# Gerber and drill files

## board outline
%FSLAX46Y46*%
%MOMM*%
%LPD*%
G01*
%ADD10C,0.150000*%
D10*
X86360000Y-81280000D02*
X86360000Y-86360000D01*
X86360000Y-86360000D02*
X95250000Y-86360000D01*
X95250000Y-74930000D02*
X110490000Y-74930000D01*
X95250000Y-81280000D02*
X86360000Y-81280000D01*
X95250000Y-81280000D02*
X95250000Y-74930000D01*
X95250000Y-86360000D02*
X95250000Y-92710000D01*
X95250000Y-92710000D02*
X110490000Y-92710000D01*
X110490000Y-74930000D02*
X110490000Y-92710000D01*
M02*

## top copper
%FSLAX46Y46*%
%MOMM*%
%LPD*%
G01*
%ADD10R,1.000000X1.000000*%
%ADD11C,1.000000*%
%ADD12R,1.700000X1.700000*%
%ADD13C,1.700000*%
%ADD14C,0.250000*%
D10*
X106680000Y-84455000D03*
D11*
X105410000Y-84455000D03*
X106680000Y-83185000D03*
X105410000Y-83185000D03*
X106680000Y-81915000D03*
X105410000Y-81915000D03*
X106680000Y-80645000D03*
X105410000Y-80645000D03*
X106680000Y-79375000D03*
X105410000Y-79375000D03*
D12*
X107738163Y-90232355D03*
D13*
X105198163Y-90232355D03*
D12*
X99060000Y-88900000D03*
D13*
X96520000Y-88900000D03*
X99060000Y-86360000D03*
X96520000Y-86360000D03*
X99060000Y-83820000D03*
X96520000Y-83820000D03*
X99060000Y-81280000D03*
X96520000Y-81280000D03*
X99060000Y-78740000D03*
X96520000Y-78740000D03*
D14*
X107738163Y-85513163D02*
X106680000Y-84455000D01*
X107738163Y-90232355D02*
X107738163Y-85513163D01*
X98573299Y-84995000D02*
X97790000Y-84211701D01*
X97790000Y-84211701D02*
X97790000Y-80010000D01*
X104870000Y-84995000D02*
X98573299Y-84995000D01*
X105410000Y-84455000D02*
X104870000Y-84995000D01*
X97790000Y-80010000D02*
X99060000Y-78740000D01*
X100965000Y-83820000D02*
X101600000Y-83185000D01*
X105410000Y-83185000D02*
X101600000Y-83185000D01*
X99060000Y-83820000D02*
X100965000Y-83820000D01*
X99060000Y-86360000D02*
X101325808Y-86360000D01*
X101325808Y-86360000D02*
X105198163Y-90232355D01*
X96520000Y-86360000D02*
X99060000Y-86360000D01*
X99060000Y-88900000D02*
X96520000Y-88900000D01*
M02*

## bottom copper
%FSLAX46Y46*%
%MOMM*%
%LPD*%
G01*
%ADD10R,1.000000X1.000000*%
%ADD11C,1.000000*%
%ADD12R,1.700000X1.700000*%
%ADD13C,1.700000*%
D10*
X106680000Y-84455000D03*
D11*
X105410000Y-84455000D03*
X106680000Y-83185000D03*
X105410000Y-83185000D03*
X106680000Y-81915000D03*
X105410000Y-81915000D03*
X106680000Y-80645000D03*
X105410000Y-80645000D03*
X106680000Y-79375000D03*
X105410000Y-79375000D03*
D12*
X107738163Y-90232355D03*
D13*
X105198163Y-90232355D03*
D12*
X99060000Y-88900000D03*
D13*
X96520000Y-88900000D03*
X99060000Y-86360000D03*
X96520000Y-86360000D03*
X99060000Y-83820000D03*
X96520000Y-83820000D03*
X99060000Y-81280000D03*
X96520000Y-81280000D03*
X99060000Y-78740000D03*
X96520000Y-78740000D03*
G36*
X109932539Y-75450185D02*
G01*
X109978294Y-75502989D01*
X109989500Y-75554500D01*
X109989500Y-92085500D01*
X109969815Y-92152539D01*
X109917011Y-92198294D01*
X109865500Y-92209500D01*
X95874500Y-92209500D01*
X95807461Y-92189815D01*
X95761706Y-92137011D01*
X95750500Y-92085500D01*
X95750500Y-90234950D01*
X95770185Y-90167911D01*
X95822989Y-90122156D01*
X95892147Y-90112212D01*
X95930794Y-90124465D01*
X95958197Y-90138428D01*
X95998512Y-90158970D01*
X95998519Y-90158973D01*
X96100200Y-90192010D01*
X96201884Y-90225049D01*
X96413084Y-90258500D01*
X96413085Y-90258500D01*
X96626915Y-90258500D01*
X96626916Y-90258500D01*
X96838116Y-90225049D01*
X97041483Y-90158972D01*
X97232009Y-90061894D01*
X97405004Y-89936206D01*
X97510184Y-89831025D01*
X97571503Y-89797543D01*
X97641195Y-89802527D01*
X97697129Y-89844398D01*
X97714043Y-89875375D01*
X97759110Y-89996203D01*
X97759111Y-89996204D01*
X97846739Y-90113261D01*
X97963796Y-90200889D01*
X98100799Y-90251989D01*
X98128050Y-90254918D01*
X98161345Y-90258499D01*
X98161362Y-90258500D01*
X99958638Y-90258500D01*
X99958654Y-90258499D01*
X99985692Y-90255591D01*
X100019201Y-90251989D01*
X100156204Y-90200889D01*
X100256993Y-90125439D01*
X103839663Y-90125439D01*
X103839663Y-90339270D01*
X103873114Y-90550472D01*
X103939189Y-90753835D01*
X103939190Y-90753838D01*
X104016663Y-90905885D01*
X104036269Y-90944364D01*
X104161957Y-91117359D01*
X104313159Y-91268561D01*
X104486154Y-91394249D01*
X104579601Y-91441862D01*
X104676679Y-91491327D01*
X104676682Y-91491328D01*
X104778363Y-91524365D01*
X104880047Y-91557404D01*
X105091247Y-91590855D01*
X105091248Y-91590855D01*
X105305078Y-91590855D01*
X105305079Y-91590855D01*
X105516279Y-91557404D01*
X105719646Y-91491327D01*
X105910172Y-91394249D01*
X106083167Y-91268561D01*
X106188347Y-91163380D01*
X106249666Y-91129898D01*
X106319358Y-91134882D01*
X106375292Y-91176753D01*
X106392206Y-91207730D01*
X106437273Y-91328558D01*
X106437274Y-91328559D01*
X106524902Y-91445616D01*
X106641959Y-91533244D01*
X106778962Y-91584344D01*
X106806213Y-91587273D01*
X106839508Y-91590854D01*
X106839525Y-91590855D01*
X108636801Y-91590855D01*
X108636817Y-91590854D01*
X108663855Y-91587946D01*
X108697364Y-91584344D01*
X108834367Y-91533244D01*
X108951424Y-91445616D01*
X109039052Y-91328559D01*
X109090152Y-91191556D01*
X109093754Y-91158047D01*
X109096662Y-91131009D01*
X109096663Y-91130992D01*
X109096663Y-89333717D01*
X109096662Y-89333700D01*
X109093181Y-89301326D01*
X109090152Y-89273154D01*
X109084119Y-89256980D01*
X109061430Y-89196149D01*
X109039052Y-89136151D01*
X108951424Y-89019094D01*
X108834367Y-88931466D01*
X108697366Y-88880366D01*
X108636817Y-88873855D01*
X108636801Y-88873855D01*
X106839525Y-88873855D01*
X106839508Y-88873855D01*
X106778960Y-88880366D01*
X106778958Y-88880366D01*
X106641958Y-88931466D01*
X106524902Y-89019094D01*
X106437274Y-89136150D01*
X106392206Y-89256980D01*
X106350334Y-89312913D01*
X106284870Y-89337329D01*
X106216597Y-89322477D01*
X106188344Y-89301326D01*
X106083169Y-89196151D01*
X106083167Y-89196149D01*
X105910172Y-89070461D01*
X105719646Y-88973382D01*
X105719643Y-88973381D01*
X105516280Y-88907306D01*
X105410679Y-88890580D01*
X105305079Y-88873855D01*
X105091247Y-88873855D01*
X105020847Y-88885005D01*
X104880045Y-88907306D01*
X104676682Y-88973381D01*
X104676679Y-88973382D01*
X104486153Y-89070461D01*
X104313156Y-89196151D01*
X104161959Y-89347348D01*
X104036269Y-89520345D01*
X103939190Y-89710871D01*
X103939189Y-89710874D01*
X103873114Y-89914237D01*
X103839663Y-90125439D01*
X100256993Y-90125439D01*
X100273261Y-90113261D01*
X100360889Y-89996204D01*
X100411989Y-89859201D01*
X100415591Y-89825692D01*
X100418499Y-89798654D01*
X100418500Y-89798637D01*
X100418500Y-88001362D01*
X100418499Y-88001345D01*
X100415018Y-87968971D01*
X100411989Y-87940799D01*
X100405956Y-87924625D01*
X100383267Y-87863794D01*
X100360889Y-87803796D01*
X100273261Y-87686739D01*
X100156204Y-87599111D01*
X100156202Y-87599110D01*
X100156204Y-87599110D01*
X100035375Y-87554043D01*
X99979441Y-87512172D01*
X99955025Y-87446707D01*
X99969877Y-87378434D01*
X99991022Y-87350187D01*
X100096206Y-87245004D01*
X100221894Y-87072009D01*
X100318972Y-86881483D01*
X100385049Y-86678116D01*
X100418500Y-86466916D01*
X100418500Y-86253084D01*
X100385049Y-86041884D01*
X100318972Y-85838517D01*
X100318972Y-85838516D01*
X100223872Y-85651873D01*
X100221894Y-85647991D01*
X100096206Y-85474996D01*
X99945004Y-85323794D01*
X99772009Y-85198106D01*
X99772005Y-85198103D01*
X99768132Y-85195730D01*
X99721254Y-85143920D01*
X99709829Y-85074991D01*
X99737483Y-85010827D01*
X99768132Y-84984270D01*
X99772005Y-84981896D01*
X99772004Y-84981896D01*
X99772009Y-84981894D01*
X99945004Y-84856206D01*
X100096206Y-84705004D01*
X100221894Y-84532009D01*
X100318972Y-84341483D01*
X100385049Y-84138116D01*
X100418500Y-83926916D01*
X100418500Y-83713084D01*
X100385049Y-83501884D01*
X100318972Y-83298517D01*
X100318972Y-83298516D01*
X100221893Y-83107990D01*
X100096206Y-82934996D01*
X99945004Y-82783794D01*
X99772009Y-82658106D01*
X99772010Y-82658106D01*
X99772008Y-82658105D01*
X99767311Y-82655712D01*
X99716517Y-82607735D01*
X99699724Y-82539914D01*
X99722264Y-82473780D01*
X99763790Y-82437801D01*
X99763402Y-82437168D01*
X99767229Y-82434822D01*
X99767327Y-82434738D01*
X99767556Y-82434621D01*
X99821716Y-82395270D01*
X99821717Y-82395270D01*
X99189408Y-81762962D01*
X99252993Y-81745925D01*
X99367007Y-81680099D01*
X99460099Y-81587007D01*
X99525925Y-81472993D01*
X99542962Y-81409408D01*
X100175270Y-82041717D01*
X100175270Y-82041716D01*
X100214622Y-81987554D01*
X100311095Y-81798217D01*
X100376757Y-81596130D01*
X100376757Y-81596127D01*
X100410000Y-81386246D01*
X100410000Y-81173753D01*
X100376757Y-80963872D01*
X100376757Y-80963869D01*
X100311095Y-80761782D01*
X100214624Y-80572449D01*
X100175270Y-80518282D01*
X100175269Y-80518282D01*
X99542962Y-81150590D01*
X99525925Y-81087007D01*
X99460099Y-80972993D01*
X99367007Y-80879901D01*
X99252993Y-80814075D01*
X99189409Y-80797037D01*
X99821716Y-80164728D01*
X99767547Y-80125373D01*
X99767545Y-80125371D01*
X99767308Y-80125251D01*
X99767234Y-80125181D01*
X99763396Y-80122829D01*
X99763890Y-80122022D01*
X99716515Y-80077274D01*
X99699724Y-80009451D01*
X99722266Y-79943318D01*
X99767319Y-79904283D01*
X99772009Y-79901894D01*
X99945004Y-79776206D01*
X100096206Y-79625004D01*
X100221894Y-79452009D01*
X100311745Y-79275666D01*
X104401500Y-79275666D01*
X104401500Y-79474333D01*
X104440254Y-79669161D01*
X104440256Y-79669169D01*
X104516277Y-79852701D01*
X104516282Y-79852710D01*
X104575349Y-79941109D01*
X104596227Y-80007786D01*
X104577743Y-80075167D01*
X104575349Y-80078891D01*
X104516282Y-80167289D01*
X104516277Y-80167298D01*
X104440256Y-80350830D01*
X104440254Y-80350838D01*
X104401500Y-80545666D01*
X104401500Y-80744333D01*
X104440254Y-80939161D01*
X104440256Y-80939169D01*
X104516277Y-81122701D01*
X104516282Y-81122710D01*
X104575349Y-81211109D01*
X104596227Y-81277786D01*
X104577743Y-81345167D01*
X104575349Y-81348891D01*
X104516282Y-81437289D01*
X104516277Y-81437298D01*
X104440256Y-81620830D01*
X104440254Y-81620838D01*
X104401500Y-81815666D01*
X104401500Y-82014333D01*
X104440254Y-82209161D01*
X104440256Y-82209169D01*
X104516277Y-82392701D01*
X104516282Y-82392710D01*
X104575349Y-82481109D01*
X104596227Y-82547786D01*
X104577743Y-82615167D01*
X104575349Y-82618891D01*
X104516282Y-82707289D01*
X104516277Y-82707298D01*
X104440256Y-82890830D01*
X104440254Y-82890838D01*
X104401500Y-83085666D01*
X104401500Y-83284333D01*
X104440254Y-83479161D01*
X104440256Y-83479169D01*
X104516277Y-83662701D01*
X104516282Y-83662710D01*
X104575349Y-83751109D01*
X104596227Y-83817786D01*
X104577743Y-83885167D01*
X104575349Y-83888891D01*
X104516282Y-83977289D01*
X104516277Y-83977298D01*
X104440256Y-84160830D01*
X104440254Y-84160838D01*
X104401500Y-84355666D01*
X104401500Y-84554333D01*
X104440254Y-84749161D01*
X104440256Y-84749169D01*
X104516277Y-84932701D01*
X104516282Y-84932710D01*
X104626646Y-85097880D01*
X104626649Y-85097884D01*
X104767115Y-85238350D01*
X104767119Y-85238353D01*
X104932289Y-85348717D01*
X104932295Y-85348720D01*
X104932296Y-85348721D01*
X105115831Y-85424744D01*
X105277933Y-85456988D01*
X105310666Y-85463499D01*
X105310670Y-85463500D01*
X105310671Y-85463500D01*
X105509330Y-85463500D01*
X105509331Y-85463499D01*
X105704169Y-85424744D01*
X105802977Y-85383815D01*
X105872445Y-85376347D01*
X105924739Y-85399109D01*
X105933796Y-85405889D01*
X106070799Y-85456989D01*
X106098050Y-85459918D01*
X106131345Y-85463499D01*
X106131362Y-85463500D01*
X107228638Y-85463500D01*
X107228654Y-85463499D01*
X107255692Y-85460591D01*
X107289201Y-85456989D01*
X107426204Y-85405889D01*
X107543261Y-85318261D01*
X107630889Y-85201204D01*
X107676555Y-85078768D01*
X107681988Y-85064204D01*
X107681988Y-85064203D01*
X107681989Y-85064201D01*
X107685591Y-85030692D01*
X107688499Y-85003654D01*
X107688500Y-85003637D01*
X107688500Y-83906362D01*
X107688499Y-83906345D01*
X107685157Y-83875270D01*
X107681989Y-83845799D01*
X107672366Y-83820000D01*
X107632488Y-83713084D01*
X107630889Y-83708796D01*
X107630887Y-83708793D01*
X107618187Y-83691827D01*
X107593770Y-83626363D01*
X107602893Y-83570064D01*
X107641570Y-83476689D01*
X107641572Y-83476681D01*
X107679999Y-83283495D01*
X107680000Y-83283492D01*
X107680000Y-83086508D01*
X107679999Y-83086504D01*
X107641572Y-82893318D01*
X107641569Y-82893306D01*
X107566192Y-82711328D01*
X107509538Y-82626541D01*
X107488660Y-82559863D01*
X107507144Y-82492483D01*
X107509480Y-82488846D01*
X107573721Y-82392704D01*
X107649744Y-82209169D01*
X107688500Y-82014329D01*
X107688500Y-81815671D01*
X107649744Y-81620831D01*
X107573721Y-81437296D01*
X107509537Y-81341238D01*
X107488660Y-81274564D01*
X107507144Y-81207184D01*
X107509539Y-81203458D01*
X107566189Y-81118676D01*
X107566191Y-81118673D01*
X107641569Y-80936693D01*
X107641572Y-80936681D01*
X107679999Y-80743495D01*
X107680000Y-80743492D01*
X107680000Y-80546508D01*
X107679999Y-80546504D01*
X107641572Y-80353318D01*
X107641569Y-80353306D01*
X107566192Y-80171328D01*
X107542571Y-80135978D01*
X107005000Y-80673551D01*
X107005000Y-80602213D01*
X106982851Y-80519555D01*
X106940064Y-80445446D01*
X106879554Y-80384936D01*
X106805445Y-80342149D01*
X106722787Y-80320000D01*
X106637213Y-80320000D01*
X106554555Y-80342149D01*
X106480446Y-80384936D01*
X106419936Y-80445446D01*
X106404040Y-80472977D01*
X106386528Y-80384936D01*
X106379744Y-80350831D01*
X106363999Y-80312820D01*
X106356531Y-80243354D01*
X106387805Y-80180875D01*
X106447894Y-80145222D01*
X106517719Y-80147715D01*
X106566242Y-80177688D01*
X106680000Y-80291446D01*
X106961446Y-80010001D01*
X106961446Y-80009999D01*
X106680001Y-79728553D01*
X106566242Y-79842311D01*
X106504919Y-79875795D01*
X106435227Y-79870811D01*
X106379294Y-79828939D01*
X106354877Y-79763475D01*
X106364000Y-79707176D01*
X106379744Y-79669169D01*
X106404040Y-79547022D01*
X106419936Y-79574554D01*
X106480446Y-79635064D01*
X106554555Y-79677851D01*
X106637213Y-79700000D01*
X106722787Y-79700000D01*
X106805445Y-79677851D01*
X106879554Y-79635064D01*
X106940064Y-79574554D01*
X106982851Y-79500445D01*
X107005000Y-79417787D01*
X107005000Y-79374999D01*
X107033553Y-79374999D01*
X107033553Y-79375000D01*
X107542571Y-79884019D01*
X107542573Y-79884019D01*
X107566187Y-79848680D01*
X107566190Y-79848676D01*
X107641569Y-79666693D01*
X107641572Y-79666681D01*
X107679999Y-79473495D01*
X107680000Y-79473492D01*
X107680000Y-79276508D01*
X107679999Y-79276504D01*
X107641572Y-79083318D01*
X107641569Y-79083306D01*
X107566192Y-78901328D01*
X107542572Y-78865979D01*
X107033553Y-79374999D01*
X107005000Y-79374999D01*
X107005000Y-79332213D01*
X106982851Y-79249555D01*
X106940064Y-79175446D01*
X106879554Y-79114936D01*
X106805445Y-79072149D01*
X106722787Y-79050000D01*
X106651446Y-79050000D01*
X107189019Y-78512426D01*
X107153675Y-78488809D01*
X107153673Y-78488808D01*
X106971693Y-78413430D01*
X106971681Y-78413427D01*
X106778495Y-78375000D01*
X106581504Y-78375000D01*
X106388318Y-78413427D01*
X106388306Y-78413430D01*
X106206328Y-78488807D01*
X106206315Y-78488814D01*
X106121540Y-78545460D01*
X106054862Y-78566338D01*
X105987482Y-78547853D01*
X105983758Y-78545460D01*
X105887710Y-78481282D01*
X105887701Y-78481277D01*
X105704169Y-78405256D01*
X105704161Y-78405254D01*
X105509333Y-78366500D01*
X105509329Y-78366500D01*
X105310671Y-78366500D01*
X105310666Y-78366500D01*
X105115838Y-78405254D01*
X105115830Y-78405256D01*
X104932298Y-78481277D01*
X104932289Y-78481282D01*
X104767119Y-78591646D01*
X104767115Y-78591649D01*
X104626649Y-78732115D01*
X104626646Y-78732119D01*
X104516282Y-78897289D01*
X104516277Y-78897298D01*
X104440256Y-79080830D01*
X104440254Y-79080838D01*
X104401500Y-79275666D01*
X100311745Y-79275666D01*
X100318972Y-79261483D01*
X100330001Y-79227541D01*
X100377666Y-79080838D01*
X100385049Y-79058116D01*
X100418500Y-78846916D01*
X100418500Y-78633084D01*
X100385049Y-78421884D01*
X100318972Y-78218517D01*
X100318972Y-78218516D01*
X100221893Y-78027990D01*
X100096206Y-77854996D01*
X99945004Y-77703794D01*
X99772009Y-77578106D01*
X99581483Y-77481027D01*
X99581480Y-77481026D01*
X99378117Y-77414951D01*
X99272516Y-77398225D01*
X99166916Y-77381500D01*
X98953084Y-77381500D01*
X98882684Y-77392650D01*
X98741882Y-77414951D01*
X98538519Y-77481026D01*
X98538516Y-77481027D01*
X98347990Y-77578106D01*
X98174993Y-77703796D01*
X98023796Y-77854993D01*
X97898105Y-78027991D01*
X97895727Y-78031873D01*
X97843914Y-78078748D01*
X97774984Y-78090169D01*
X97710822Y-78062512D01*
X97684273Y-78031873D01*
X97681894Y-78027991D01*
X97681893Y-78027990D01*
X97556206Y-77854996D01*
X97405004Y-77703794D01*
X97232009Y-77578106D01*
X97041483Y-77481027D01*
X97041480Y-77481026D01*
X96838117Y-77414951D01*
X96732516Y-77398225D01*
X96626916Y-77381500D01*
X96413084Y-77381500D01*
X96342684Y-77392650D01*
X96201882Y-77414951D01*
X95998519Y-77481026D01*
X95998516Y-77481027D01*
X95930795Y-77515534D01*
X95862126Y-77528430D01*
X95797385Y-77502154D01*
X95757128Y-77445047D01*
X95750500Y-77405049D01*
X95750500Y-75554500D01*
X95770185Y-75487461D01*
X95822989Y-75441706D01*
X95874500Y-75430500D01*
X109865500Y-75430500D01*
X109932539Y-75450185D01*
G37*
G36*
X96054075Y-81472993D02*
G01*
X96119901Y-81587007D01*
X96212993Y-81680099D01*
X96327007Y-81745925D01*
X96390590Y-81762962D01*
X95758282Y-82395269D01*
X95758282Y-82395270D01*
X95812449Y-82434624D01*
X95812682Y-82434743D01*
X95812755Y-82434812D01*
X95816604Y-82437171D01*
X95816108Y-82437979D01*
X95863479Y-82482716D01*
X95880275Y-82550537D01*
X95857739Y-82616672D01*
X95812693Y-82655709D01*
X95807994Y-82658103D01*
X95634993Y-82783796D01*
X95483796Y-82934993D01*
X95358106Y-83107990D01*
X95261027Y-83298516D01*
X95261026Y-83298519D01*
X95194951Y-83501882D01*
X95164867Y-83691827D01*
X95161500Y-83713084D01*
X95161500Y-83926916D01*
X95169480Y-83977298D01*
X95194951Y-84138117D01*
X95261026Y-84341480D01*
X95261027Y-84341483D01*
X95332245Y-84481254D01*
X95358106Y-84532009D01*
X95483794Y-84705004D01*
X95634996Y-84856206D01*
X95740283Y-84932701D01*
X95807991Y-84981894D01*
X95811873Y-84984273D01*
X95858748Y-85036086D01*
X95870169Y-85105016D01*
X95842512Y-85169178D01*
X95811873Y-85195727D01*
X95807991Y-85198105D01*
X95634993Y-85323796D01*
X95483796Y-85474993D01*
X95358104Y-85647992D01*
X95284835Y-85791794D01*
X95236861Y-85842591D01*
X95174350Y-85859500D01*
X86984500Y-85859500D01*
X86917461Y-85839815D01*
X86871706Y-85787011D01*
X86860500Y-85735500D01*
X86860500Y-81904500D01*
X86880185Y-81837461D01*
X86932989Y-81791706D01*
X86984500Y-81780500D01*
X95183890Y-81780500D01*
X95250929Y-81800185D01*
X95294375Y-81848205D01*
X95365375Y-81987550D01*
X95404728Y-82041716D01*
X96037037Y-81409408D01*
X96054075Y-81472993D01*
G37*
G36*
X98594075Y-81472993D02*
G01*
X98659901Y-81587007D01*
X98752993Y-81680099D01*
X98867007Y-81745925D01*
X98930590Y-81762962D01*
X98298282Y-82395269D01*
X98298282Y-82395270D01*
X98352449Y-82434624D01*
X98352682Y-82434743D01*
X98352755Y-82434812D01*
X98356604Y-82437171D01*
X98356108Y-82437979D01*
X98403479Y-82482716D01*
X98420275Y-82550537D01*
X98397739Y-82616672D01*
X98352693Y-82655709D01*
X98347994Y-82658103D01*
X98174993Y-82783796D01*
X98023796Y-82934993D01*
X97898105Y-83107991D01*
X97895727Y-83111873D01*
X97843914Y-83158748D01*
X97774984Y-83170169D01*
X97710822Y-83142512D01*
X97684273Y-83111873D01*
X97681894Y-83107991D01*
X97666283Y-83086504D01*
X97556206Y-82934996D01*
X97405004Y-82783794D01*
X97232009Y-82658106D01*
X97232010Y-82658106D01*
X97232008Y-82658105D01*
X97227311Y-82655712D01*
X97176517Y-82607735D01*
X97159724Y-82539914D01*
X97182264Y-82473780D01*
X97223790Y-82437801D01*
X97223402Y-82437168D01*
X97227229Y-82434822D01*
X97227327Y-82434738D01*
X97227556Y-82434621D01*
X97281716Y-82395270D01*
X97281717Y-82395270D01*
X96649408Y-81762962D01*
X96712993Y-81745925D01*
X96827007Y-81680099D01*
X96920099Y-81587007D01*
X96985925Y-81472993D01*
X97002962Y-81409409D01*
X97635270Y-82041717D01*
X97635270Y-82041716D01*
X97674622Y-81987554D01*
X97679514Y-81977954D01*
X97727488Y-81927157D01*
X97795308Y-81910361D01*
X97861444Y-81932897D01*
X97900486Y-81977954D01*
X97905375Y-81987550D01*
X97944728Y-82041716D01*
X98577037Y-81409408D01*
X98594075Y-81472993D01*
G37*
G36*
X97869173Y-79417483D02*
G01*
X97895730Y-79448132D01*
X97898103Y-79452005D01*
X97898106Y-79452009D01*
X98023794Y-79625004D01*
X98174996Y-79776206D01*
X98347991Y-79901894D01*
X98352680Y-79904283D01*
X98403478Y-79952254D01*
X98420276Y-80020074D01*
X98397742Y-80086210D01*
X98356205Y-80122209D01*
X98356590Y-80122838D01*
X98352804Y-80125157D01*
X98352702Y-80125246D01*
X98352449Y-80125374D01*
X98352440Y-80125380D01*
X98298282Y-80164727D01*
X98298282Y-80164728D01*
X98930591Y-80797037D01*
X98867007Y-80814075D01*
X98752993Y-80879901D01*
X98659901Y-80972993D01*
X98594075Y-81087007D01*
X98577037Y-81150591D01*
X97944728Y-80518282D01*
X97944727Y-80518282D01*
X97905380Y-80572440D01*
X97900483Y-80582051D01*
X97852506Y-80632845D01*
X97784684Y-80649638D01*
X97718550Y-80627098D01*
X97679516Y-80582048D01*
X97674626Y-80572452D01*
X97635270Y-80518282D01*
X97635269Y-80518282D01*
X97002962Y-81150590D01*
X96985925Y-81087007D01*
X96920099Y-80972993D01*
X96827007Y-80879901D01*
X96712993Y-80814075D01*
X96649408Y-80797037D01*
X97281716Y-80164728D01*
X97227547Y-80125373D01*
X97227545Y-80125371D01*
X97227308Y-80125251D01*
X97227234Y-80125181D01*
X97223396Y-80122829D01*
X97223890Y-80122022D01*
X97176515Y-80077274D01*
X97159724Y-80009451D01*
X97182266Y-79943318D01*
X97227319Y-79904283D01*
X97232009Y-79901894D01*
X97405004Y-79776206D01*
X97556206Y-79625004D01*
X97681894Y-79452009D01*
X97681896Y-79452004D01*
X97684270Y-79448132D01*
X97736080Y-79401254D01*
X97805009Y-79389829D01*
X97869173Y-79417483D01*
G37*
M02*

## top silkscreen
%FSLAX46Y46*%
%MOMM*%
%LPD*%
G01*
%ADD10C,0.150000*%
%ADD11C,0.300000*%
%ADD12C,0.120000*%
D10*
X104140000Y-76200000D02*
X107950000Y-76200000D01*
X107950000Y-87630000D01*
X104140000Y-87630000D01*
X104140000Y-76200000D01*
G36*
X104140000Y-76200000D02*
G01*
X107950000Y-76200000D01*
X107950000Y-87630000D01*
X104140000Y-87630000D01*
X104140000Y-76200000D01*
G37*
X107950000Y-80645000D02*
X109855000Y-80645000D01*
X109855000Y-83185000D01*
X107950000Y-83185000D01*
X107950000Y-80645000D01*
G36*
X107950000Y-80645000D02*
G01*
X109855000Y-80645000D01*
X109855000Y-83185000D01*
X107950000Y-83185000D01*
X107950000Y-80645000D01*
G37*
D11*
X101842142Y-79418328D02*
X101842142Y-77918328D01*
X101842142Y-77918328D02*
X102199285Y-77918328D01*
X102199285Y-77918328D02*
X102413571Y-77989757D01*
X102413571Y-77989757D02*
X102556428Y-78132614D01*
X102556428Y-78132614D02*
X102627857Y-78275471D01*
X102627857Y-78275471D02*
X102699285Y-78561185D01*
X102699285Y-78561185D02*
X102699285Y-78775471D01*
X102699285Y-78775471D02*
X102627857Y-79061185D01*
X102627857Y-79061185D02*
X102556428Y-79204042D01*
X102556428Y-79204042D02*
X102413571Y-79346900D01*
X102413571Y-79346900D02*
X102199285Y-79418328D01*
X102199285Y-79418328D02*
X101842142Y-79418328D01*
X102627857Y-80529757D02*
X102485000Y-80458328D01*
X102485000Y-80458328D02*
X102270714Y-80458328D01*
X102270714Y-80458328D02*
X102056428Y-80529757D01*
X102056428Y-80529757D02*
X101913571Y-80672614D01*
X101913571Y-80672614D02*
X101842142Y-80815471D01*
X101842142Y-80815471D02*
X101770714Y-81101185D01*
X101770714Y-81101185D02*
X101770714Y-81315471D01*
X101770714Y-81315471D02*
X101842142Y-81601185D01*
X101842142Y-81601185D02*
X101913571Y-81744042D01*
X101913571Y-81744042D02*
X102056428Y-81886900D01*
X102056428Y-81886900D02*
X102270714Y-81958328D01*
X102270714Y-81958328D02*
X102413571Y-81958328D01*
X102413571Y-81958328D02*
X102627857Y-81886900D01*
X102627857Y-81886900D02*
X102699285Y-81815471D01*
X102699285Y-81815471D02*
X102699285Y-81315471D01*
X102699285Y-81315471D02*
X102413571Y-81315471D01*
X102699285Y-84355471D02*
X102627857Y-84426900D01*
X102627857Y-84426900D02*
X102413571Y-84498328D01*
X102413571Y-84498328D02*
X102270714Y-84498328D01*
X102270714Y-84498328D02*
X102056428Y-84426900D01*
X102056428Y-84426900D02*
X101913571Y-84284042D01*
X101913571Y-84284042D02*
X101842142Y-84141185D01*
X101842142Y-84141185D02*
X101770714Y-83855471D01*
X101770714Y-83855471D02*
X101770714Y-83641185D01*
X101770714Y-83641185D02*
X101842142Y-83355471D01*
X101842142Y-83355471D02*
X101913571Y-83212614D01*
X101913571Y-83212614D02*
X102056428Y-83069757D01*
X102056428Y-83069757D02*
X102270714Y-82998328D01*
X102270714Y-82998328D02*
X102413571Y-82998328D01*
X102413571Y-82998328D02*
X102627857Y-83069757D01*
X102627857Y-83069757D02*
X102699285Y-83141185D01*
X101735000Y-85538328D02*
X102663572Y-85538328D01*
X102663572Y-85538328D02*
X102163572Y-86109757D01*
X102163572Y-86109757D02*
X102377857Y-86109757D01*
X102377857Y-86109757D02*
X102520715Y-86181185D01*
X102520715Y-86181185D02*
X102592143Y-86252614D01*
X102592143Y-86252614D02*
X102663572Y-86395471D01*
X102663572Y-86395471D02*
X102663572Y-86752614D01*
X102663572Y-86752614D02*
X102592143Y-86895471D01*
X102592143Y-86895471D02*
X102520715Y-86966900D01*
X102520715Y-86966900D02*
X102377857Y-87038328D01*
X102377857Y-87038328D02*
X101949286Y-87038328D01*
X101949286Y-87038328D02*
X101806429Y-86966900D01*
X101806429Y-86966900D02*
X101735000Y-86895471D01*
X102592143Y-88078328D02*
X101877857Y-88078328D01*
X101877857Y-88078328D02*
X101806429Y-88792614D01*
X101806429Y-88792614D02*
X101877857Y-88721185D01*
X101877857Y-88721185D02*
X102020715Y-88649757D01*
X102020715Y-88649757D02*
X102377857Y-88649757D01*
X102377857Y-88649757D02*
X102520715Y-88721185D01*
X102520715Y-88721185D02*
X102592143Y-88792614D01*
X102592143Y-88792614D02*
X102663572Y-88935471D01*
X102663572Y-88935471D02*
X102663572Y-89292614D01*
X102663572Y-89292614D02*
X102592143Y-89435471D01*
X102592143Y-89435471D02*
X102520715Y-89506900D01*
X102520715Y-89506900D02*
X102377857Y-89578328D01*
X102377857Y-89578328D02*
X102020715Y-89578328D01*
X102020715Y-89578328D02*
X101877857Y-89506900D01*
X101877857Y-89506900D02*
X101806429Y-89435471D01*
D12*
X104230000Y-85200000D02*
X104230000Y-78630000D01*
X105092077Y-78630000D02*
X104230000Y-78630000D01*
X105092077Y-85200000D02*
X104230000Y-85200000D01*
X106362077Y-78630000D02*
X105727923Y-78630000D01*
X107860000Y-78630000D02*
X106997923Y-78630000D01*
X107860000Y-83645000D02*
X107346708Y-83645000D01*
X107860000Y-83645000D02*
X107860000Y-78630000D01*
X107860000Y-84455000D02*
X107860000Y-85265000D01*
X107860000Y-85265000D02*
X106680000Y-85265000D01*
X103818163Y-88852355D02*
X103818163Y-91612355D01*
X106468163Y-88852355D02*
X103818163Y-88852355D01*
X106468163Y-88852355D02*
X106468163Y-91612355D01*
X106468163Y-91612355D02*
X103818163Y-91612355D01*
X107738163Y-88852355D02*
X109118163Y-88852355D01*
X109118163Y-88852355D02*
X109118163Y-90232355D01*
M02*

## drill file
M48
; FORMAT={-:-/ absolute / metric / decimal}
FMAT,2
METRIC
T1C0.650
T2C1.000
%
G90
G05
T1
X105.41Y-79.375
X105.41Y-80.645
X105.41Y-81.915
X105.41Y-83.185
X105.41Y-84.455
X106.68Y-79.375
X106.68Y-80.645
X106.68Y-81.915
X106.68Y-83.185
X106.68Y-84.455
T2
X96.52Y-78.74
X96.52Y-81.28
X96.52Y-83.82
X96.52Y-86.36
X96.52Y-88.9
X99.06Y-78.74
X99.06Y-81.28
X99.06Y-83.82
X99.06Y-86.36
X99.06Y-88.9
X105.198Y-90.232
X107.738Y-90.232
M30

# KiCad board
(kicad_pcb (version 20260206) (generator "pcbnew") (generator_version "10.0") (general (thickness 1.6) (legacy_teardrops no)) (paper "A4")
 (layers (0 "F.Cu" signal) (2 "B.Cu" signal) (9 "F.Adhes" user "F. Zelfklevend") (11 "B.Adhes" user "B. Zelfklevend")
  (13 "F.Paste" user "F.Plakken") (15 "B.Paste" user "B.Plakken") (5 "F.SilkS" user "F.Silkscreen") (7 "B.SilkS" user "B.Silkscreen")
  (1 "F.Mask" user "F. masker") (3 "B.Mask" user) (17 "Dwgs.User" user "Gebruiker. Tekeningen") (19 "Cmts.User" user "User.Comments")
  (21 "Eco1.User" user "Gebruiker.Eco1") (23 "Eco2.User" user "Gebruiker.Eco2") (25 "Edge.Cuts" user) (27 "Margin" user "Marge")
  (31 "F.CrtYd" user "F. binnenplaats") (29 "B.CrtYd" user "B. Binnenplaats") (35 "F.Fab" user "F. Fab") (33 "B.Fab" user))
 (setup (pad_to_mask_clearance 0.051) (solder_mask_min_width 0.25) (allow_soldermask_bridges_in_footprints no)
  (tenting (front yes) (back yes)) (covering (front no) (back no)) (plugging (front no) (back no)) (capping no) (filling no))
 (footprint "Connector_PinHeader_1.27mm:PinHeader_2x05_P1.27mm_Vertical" (layer "F.Cu") (at 106.68 84.455 180)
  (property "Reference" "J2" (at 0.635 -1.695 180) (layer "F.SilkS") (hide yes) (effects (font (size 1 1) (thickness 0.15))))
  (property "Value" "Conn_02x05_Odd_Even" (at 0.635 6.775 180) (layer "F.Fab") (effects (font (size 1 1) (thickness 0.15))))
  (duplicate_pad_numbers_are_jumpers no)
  (fp_line (start 2.45 -0.745) (end 2.45 5.825) (stroke (width 0.12) (type solid)) (layer "F.SilkS"))
  (fp_line (start 1.587923 5.825) (end 2.45 5.825) (stroke (width 0.12) (type solid)) (layer "F.SilkS"))
  (fp_line (start 1.587923 -0.745) (end 2.45 -0.745) (stroke (width 0.12) (type solid)) (layer "F.SilkS"))
  (fp_line (start 0.317923 5.825) (end 0.952077 5.825) (stroke (width 0.12) (type solid)) (layer "F.SilkS"))
  (fp_line (start -1.18 5.825) (end -0.317923 5.825) (stroke (width 0.12) (type solid)) (layer "F.SilkS"))
  (fp_line (start -1.18 0.81) (end -0.666708 0.81) (stroke (width 0.12) (type solid)) (layer "F.SilkS"))
  (fp_line (start -1.18 0.81) (end -1.18 5.825) (stroke (width 0.12) (type solid)) (layer "F.SilkS"))
  (fp_line (start -1.18 0) (end -1.18 -0.81) (stroke (width 0.12) (type solid)) (layer "F.SilkS"))
  (fp_line (start -1.18 -0.81) (end 0 -0.81) (stroke (width 0.12) (type solid)) (layer "F.SilkS"))
  (pad "1" thru_hole rect (at 0 0 180) (size 1 1) (drill 0.65) (layers "*.Cu" "*.Mask") (remove_unused_layers no) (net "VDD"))
  (pad "2" thru_hole circle (at 1.27 0 180) (size 1 1) (drill 0.65) (layers "*.Cu" "*.Mask") (remove_unused_layers no) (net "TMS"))
  (pad "3" thru_hole circle (at 0 1.27 180) (size 1 1) (drill 0.65) (layers "*.Cu" "*.Mask") (remove_unused_layers no) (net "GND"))
  (pad "4" thru_hole circle (at 1.27 1.27 180) (size 1 1) (drill 0.65) (layers "*.Cu" "*.Mask") (remove_unused_layers no) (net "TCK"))
  (pad "5" thru_hole circle (at 0 2.54 180) (size 1 1) (drill 0.65) (layers "*.Cu" "*.Mask") (remove_unused_layers no)
   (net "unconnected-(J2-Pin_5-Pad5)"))
  (pad "6" thru_hole circle (at 1.27 2.54 180) (size 1 1) (drill 0.65) (layers "*.Cu" "*.Mask") (remove_unused_layers no) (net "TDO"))
  (pad "7" thru_hole circle (at 0 3.81 180) (size 1 1) (drill 0.65) (layers "*.Cu" "*.Mask") (remove_unused_layers no) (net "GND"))
  (pad "8" thru_hole circle (at 1.27 3.81 180) (size 1 1) (drill 0.65) (layers "*.Cu" "*.Mask") (remove_unused_layers no) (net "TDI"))
  (pad "9" thru_hole circle (at 0 5.08 180) (size 1 1) (drill 0.65) (layers "*.Cu" "*.Mask") (remove_unused_layers no) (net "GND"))
  (pad "10" thru_hole circle (at 1.27 5.08 180) (size 1 1) (drill 0.65) (layers "*.Cu" "*.Mask") (remove_unused_layers no) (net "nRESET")))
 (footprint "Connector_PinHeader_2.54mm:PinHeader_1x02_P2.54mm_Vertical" (layer "F.Cu") (at 107.738163 90.232355 -90)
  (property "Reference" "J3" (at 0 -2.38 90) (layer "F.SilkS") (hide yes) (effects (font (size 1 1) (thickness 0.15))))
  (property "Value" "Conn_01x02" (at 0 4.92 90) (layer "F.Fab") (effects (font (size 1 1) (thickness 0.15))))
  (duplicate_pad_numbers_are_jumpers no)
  (fp_line (start -1.38 3.92) (end 1.38 3.92) (stroke (width 0.12) (type solid)) (layer "F.SilkS"))
  (fp_line (start -1.38 1.27) (end -1.38 3.92) (stroke (width 0.12) (type solid)) (layer "F.SilkS"))
  (fp_line (start -1.38 1.27) (end 1.38 1.27) (stroke (width 0.12) (type solid)) (layer "F.SilkS"))
  (fp_line (start 1.38 1.27) (end 1.38 3.92) (stroke (width 0.12) (type solid)) (layer "F.SilkS"))
  (fp_line (start -1.38 0) (end -1.38 -1.38) (stroke (width 0.12) (type solid)) (layer "F.SilkS"))
  (fp_line (start -1.38 -1.38) (end 0 -1.38) (stroke (width 0.12) (type solid)) (layer "F.SilkS"))
  (pad "1" thru_hole rect (at 0 0 270) (size 1.7 1.7) (drill 1) (layers "*.Cu" "*.Mask") (remove_unused_layers no) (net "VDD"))
  (pad "2" thru_hole circle (at 0 2.54 270) (size 1.7 1.7) (drill 1) (layers "*.Cu" "*.Mask") (remove_unused_layers no) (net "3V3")))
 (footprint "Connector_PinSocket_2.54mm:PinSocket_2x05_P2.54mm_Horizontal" (layer "B.Cu") (at 99.06 88.9)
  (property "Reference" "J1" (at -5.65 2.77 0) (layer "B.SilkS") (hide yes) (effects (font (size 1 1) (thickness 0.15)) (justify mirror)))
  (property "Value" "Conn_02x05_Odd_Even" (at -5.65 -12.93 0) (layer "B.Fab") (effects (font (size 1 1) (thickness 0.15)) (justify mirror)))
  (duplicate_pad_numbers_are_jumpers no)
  (pad "1" thru_hole rect (at 0 0) (size 1.7 1.7) (drill 1) (layers "*.Cu" "*.Mask") (remove_unused_layers no) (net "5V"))
  (pad "2" thru_hole circle (at -2.54 0) (size 1.7 1.7) (drill 1) (layers "*.Cu" "*.Mask") (remove_unused_layers no) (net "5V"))
  (pad "3" thru_hole circle (at 0 -2.54) (size 1.7 1.7) (drill 1) (layers "*.Cu" "*.Mask") (remove_unused_layers no) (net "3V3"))
  (pad "4" thru_hole circle (at -2.54 -2.54) (size 1.7 1.7) (drill 1) (layers "*.Cu" "*.Mask") (remove_unused_layers no) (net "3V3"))
  (pad "5" thru_hole circle (at 0 -5.08) (size 1.7 1.7) (drill 1) (layers "*.Cu" "*.Mask") (remove_unused_layers no) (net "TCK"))
  (pad "6" thru_hole circle (at -2.54 -5.08) (size 1.7 1.7) (drill 1) (layers "*.Cu" "*.Mask") (remove_unused_layers no) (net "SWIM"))
  (pad "7" thru_hole circle (at 0 -7.62) (size 1.7 1.7) (drill 1) (layers "*.Cu" "*.Mask") (remove_unused_layers no) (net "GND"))
  (pad "8" thru_hole circle (at -2.54 -7.62) (size 1.7 1.7) (drill 1) (layers "*.Cu" "*.Mask") (remove_unused_layers no) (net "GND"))
  (pad "9" thru_hole circle (at 0 -10.16) (size 1.7 1.7) (drill 1) (layers "*.Cu" "*.Mask") (remove_unused_layers no) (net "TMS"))
  (pad "10" thru_hole circle (at -2.54 -10.16) (size 1.7 1.7) (drill 1) (layers "*.Cu" "*.Mask") (remove_unused_layers no)
   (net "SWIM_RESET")))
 (gr_rect (start 104.14 76.2) (end 107.95 87.63) (stroke (width 0.15) (type solid)) (fill yes) (layer "F.SilkS"))
 (gr_rect (start 107.95 80.645) (end 109.855 83.185) (stroke (width 0.15) (type solid)) (fill yes) (layer "F.SilkS"))
 (gr_line (start 86.36 81.28) (end 86.36 86.36) (stroke (width 0.15) (type default)) (layer "Edge.Cuts"))
 (gr_line (start 86.36 86.36) (end 95.25 86.36) (stroke (width 0.15) (type default)) (layer "Edge.Cuts"))
 (gr_line (start 95.25 74.93) (end 110.49 74.93) (stroke (width 0.15) (type default)) (layer "Edge.Cuts"))
 (gr_line (start 95.25 81.28) (end 86.36 81.28) (stroke (width 0.15) (type default)) (layer "Edge.Cuts"))
 (gr_line (start 95.25 81.28) (end 95.25 74.93) (stroke (width 0.15) (type default)) (layer "Edge.Cuts"))
 (gr_line (start 95.25 86.36) (end 95.25 92.71) (stroke (width 0.15) (type default)) (layer "Edge.Cuts"))
 (gr_line (start 95.25 92.71) (end 110.49 92.71) (stroke (width 0.15) (type default)) (layer "Edge.Cuts"))
 (gr_line (start 110.49 74.93) (end 110.49 92.71) (stroke (width 0.15) (type default)) (layer "Edge.Cuts"))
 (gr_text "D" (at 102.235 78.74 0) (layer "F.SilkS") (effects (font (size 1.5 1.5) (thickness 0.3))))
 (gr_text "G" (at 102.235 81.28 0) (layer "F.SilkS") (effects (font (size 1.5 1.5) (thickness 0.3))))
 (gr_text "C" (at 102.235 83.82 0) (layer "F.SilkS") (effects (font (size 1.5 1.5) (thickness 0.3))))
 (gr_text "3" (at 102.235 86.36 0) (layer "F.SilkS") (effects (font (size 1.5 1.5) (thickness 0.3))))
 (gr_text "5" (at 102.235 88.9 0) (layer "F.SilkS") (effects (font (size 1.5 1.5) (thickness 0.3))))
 (segment (start 107.738163 85.513163) (end 106.68 84.455) (width 0.25) (layer "F.Cu") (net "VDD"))
 (segment (start 107.738163 90.232355) (end 107.738163 85.513163) (width 0.25) (layer "F.Cu") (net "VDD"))
 (segment (start 98.573299 84.995) (end 97.79 84.211701) (width 0.25) (layer "F.Cu") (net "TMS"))
 (segment (start 97.79 84.211701) (end 97.79 80.01) (width 0.25) (layer "F.Cu") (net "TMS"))
 (segment (start 104.87 84.995) (end 98.573299 84.995) (width 0.25) (layer "F.Cu") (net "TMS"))
 (segment (start 105.41 84.455) (end 104.87 84.995) (width 0.25) (layer "F.Cu") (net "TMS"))
 (segment (start 97.79 80.01) (end 99.06 78.74) (width 0.25) (layer "F.Cu") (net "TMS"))
 (segment (start 100.965 83.82) (end 101.6 83.185) (width 0.25) (layer "F.Cu") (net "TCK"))
 (segment (start 105.41 83.185) (end 101.6 83.185) (width 0.25) (layer "F.Cu") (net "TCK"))
 (segment (start 99.06 83.82) (end 100.965 83.82) (width 0.25) (layer "F.Cu") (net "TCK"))
 (segment (start 99.06 86.36) (end 101.325808 86.36) (width 0.25) (layer "F.Cu") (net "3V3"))
 (segment (start 101.325808 86.36) (end 105.198163 90.232355) (width 0.25) (layer "F.Cu") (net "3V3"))
 (segment (start 96.52 86.36) (end 99.06 86.36) (width 0.25) (layer "F.Cu") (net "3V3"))
 (segment (start 99.06 88.9) (end 96.52 88.9) (width 0.25) (layer "F.Cu") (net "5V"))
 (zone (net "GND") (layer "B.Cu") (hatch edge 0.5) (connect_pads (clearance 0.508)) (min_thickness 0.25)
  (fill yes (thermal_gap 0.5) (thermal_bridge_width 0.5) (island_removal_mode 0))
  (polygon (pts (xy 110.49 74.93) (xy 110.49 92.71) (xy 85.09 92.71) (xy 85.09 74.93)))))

